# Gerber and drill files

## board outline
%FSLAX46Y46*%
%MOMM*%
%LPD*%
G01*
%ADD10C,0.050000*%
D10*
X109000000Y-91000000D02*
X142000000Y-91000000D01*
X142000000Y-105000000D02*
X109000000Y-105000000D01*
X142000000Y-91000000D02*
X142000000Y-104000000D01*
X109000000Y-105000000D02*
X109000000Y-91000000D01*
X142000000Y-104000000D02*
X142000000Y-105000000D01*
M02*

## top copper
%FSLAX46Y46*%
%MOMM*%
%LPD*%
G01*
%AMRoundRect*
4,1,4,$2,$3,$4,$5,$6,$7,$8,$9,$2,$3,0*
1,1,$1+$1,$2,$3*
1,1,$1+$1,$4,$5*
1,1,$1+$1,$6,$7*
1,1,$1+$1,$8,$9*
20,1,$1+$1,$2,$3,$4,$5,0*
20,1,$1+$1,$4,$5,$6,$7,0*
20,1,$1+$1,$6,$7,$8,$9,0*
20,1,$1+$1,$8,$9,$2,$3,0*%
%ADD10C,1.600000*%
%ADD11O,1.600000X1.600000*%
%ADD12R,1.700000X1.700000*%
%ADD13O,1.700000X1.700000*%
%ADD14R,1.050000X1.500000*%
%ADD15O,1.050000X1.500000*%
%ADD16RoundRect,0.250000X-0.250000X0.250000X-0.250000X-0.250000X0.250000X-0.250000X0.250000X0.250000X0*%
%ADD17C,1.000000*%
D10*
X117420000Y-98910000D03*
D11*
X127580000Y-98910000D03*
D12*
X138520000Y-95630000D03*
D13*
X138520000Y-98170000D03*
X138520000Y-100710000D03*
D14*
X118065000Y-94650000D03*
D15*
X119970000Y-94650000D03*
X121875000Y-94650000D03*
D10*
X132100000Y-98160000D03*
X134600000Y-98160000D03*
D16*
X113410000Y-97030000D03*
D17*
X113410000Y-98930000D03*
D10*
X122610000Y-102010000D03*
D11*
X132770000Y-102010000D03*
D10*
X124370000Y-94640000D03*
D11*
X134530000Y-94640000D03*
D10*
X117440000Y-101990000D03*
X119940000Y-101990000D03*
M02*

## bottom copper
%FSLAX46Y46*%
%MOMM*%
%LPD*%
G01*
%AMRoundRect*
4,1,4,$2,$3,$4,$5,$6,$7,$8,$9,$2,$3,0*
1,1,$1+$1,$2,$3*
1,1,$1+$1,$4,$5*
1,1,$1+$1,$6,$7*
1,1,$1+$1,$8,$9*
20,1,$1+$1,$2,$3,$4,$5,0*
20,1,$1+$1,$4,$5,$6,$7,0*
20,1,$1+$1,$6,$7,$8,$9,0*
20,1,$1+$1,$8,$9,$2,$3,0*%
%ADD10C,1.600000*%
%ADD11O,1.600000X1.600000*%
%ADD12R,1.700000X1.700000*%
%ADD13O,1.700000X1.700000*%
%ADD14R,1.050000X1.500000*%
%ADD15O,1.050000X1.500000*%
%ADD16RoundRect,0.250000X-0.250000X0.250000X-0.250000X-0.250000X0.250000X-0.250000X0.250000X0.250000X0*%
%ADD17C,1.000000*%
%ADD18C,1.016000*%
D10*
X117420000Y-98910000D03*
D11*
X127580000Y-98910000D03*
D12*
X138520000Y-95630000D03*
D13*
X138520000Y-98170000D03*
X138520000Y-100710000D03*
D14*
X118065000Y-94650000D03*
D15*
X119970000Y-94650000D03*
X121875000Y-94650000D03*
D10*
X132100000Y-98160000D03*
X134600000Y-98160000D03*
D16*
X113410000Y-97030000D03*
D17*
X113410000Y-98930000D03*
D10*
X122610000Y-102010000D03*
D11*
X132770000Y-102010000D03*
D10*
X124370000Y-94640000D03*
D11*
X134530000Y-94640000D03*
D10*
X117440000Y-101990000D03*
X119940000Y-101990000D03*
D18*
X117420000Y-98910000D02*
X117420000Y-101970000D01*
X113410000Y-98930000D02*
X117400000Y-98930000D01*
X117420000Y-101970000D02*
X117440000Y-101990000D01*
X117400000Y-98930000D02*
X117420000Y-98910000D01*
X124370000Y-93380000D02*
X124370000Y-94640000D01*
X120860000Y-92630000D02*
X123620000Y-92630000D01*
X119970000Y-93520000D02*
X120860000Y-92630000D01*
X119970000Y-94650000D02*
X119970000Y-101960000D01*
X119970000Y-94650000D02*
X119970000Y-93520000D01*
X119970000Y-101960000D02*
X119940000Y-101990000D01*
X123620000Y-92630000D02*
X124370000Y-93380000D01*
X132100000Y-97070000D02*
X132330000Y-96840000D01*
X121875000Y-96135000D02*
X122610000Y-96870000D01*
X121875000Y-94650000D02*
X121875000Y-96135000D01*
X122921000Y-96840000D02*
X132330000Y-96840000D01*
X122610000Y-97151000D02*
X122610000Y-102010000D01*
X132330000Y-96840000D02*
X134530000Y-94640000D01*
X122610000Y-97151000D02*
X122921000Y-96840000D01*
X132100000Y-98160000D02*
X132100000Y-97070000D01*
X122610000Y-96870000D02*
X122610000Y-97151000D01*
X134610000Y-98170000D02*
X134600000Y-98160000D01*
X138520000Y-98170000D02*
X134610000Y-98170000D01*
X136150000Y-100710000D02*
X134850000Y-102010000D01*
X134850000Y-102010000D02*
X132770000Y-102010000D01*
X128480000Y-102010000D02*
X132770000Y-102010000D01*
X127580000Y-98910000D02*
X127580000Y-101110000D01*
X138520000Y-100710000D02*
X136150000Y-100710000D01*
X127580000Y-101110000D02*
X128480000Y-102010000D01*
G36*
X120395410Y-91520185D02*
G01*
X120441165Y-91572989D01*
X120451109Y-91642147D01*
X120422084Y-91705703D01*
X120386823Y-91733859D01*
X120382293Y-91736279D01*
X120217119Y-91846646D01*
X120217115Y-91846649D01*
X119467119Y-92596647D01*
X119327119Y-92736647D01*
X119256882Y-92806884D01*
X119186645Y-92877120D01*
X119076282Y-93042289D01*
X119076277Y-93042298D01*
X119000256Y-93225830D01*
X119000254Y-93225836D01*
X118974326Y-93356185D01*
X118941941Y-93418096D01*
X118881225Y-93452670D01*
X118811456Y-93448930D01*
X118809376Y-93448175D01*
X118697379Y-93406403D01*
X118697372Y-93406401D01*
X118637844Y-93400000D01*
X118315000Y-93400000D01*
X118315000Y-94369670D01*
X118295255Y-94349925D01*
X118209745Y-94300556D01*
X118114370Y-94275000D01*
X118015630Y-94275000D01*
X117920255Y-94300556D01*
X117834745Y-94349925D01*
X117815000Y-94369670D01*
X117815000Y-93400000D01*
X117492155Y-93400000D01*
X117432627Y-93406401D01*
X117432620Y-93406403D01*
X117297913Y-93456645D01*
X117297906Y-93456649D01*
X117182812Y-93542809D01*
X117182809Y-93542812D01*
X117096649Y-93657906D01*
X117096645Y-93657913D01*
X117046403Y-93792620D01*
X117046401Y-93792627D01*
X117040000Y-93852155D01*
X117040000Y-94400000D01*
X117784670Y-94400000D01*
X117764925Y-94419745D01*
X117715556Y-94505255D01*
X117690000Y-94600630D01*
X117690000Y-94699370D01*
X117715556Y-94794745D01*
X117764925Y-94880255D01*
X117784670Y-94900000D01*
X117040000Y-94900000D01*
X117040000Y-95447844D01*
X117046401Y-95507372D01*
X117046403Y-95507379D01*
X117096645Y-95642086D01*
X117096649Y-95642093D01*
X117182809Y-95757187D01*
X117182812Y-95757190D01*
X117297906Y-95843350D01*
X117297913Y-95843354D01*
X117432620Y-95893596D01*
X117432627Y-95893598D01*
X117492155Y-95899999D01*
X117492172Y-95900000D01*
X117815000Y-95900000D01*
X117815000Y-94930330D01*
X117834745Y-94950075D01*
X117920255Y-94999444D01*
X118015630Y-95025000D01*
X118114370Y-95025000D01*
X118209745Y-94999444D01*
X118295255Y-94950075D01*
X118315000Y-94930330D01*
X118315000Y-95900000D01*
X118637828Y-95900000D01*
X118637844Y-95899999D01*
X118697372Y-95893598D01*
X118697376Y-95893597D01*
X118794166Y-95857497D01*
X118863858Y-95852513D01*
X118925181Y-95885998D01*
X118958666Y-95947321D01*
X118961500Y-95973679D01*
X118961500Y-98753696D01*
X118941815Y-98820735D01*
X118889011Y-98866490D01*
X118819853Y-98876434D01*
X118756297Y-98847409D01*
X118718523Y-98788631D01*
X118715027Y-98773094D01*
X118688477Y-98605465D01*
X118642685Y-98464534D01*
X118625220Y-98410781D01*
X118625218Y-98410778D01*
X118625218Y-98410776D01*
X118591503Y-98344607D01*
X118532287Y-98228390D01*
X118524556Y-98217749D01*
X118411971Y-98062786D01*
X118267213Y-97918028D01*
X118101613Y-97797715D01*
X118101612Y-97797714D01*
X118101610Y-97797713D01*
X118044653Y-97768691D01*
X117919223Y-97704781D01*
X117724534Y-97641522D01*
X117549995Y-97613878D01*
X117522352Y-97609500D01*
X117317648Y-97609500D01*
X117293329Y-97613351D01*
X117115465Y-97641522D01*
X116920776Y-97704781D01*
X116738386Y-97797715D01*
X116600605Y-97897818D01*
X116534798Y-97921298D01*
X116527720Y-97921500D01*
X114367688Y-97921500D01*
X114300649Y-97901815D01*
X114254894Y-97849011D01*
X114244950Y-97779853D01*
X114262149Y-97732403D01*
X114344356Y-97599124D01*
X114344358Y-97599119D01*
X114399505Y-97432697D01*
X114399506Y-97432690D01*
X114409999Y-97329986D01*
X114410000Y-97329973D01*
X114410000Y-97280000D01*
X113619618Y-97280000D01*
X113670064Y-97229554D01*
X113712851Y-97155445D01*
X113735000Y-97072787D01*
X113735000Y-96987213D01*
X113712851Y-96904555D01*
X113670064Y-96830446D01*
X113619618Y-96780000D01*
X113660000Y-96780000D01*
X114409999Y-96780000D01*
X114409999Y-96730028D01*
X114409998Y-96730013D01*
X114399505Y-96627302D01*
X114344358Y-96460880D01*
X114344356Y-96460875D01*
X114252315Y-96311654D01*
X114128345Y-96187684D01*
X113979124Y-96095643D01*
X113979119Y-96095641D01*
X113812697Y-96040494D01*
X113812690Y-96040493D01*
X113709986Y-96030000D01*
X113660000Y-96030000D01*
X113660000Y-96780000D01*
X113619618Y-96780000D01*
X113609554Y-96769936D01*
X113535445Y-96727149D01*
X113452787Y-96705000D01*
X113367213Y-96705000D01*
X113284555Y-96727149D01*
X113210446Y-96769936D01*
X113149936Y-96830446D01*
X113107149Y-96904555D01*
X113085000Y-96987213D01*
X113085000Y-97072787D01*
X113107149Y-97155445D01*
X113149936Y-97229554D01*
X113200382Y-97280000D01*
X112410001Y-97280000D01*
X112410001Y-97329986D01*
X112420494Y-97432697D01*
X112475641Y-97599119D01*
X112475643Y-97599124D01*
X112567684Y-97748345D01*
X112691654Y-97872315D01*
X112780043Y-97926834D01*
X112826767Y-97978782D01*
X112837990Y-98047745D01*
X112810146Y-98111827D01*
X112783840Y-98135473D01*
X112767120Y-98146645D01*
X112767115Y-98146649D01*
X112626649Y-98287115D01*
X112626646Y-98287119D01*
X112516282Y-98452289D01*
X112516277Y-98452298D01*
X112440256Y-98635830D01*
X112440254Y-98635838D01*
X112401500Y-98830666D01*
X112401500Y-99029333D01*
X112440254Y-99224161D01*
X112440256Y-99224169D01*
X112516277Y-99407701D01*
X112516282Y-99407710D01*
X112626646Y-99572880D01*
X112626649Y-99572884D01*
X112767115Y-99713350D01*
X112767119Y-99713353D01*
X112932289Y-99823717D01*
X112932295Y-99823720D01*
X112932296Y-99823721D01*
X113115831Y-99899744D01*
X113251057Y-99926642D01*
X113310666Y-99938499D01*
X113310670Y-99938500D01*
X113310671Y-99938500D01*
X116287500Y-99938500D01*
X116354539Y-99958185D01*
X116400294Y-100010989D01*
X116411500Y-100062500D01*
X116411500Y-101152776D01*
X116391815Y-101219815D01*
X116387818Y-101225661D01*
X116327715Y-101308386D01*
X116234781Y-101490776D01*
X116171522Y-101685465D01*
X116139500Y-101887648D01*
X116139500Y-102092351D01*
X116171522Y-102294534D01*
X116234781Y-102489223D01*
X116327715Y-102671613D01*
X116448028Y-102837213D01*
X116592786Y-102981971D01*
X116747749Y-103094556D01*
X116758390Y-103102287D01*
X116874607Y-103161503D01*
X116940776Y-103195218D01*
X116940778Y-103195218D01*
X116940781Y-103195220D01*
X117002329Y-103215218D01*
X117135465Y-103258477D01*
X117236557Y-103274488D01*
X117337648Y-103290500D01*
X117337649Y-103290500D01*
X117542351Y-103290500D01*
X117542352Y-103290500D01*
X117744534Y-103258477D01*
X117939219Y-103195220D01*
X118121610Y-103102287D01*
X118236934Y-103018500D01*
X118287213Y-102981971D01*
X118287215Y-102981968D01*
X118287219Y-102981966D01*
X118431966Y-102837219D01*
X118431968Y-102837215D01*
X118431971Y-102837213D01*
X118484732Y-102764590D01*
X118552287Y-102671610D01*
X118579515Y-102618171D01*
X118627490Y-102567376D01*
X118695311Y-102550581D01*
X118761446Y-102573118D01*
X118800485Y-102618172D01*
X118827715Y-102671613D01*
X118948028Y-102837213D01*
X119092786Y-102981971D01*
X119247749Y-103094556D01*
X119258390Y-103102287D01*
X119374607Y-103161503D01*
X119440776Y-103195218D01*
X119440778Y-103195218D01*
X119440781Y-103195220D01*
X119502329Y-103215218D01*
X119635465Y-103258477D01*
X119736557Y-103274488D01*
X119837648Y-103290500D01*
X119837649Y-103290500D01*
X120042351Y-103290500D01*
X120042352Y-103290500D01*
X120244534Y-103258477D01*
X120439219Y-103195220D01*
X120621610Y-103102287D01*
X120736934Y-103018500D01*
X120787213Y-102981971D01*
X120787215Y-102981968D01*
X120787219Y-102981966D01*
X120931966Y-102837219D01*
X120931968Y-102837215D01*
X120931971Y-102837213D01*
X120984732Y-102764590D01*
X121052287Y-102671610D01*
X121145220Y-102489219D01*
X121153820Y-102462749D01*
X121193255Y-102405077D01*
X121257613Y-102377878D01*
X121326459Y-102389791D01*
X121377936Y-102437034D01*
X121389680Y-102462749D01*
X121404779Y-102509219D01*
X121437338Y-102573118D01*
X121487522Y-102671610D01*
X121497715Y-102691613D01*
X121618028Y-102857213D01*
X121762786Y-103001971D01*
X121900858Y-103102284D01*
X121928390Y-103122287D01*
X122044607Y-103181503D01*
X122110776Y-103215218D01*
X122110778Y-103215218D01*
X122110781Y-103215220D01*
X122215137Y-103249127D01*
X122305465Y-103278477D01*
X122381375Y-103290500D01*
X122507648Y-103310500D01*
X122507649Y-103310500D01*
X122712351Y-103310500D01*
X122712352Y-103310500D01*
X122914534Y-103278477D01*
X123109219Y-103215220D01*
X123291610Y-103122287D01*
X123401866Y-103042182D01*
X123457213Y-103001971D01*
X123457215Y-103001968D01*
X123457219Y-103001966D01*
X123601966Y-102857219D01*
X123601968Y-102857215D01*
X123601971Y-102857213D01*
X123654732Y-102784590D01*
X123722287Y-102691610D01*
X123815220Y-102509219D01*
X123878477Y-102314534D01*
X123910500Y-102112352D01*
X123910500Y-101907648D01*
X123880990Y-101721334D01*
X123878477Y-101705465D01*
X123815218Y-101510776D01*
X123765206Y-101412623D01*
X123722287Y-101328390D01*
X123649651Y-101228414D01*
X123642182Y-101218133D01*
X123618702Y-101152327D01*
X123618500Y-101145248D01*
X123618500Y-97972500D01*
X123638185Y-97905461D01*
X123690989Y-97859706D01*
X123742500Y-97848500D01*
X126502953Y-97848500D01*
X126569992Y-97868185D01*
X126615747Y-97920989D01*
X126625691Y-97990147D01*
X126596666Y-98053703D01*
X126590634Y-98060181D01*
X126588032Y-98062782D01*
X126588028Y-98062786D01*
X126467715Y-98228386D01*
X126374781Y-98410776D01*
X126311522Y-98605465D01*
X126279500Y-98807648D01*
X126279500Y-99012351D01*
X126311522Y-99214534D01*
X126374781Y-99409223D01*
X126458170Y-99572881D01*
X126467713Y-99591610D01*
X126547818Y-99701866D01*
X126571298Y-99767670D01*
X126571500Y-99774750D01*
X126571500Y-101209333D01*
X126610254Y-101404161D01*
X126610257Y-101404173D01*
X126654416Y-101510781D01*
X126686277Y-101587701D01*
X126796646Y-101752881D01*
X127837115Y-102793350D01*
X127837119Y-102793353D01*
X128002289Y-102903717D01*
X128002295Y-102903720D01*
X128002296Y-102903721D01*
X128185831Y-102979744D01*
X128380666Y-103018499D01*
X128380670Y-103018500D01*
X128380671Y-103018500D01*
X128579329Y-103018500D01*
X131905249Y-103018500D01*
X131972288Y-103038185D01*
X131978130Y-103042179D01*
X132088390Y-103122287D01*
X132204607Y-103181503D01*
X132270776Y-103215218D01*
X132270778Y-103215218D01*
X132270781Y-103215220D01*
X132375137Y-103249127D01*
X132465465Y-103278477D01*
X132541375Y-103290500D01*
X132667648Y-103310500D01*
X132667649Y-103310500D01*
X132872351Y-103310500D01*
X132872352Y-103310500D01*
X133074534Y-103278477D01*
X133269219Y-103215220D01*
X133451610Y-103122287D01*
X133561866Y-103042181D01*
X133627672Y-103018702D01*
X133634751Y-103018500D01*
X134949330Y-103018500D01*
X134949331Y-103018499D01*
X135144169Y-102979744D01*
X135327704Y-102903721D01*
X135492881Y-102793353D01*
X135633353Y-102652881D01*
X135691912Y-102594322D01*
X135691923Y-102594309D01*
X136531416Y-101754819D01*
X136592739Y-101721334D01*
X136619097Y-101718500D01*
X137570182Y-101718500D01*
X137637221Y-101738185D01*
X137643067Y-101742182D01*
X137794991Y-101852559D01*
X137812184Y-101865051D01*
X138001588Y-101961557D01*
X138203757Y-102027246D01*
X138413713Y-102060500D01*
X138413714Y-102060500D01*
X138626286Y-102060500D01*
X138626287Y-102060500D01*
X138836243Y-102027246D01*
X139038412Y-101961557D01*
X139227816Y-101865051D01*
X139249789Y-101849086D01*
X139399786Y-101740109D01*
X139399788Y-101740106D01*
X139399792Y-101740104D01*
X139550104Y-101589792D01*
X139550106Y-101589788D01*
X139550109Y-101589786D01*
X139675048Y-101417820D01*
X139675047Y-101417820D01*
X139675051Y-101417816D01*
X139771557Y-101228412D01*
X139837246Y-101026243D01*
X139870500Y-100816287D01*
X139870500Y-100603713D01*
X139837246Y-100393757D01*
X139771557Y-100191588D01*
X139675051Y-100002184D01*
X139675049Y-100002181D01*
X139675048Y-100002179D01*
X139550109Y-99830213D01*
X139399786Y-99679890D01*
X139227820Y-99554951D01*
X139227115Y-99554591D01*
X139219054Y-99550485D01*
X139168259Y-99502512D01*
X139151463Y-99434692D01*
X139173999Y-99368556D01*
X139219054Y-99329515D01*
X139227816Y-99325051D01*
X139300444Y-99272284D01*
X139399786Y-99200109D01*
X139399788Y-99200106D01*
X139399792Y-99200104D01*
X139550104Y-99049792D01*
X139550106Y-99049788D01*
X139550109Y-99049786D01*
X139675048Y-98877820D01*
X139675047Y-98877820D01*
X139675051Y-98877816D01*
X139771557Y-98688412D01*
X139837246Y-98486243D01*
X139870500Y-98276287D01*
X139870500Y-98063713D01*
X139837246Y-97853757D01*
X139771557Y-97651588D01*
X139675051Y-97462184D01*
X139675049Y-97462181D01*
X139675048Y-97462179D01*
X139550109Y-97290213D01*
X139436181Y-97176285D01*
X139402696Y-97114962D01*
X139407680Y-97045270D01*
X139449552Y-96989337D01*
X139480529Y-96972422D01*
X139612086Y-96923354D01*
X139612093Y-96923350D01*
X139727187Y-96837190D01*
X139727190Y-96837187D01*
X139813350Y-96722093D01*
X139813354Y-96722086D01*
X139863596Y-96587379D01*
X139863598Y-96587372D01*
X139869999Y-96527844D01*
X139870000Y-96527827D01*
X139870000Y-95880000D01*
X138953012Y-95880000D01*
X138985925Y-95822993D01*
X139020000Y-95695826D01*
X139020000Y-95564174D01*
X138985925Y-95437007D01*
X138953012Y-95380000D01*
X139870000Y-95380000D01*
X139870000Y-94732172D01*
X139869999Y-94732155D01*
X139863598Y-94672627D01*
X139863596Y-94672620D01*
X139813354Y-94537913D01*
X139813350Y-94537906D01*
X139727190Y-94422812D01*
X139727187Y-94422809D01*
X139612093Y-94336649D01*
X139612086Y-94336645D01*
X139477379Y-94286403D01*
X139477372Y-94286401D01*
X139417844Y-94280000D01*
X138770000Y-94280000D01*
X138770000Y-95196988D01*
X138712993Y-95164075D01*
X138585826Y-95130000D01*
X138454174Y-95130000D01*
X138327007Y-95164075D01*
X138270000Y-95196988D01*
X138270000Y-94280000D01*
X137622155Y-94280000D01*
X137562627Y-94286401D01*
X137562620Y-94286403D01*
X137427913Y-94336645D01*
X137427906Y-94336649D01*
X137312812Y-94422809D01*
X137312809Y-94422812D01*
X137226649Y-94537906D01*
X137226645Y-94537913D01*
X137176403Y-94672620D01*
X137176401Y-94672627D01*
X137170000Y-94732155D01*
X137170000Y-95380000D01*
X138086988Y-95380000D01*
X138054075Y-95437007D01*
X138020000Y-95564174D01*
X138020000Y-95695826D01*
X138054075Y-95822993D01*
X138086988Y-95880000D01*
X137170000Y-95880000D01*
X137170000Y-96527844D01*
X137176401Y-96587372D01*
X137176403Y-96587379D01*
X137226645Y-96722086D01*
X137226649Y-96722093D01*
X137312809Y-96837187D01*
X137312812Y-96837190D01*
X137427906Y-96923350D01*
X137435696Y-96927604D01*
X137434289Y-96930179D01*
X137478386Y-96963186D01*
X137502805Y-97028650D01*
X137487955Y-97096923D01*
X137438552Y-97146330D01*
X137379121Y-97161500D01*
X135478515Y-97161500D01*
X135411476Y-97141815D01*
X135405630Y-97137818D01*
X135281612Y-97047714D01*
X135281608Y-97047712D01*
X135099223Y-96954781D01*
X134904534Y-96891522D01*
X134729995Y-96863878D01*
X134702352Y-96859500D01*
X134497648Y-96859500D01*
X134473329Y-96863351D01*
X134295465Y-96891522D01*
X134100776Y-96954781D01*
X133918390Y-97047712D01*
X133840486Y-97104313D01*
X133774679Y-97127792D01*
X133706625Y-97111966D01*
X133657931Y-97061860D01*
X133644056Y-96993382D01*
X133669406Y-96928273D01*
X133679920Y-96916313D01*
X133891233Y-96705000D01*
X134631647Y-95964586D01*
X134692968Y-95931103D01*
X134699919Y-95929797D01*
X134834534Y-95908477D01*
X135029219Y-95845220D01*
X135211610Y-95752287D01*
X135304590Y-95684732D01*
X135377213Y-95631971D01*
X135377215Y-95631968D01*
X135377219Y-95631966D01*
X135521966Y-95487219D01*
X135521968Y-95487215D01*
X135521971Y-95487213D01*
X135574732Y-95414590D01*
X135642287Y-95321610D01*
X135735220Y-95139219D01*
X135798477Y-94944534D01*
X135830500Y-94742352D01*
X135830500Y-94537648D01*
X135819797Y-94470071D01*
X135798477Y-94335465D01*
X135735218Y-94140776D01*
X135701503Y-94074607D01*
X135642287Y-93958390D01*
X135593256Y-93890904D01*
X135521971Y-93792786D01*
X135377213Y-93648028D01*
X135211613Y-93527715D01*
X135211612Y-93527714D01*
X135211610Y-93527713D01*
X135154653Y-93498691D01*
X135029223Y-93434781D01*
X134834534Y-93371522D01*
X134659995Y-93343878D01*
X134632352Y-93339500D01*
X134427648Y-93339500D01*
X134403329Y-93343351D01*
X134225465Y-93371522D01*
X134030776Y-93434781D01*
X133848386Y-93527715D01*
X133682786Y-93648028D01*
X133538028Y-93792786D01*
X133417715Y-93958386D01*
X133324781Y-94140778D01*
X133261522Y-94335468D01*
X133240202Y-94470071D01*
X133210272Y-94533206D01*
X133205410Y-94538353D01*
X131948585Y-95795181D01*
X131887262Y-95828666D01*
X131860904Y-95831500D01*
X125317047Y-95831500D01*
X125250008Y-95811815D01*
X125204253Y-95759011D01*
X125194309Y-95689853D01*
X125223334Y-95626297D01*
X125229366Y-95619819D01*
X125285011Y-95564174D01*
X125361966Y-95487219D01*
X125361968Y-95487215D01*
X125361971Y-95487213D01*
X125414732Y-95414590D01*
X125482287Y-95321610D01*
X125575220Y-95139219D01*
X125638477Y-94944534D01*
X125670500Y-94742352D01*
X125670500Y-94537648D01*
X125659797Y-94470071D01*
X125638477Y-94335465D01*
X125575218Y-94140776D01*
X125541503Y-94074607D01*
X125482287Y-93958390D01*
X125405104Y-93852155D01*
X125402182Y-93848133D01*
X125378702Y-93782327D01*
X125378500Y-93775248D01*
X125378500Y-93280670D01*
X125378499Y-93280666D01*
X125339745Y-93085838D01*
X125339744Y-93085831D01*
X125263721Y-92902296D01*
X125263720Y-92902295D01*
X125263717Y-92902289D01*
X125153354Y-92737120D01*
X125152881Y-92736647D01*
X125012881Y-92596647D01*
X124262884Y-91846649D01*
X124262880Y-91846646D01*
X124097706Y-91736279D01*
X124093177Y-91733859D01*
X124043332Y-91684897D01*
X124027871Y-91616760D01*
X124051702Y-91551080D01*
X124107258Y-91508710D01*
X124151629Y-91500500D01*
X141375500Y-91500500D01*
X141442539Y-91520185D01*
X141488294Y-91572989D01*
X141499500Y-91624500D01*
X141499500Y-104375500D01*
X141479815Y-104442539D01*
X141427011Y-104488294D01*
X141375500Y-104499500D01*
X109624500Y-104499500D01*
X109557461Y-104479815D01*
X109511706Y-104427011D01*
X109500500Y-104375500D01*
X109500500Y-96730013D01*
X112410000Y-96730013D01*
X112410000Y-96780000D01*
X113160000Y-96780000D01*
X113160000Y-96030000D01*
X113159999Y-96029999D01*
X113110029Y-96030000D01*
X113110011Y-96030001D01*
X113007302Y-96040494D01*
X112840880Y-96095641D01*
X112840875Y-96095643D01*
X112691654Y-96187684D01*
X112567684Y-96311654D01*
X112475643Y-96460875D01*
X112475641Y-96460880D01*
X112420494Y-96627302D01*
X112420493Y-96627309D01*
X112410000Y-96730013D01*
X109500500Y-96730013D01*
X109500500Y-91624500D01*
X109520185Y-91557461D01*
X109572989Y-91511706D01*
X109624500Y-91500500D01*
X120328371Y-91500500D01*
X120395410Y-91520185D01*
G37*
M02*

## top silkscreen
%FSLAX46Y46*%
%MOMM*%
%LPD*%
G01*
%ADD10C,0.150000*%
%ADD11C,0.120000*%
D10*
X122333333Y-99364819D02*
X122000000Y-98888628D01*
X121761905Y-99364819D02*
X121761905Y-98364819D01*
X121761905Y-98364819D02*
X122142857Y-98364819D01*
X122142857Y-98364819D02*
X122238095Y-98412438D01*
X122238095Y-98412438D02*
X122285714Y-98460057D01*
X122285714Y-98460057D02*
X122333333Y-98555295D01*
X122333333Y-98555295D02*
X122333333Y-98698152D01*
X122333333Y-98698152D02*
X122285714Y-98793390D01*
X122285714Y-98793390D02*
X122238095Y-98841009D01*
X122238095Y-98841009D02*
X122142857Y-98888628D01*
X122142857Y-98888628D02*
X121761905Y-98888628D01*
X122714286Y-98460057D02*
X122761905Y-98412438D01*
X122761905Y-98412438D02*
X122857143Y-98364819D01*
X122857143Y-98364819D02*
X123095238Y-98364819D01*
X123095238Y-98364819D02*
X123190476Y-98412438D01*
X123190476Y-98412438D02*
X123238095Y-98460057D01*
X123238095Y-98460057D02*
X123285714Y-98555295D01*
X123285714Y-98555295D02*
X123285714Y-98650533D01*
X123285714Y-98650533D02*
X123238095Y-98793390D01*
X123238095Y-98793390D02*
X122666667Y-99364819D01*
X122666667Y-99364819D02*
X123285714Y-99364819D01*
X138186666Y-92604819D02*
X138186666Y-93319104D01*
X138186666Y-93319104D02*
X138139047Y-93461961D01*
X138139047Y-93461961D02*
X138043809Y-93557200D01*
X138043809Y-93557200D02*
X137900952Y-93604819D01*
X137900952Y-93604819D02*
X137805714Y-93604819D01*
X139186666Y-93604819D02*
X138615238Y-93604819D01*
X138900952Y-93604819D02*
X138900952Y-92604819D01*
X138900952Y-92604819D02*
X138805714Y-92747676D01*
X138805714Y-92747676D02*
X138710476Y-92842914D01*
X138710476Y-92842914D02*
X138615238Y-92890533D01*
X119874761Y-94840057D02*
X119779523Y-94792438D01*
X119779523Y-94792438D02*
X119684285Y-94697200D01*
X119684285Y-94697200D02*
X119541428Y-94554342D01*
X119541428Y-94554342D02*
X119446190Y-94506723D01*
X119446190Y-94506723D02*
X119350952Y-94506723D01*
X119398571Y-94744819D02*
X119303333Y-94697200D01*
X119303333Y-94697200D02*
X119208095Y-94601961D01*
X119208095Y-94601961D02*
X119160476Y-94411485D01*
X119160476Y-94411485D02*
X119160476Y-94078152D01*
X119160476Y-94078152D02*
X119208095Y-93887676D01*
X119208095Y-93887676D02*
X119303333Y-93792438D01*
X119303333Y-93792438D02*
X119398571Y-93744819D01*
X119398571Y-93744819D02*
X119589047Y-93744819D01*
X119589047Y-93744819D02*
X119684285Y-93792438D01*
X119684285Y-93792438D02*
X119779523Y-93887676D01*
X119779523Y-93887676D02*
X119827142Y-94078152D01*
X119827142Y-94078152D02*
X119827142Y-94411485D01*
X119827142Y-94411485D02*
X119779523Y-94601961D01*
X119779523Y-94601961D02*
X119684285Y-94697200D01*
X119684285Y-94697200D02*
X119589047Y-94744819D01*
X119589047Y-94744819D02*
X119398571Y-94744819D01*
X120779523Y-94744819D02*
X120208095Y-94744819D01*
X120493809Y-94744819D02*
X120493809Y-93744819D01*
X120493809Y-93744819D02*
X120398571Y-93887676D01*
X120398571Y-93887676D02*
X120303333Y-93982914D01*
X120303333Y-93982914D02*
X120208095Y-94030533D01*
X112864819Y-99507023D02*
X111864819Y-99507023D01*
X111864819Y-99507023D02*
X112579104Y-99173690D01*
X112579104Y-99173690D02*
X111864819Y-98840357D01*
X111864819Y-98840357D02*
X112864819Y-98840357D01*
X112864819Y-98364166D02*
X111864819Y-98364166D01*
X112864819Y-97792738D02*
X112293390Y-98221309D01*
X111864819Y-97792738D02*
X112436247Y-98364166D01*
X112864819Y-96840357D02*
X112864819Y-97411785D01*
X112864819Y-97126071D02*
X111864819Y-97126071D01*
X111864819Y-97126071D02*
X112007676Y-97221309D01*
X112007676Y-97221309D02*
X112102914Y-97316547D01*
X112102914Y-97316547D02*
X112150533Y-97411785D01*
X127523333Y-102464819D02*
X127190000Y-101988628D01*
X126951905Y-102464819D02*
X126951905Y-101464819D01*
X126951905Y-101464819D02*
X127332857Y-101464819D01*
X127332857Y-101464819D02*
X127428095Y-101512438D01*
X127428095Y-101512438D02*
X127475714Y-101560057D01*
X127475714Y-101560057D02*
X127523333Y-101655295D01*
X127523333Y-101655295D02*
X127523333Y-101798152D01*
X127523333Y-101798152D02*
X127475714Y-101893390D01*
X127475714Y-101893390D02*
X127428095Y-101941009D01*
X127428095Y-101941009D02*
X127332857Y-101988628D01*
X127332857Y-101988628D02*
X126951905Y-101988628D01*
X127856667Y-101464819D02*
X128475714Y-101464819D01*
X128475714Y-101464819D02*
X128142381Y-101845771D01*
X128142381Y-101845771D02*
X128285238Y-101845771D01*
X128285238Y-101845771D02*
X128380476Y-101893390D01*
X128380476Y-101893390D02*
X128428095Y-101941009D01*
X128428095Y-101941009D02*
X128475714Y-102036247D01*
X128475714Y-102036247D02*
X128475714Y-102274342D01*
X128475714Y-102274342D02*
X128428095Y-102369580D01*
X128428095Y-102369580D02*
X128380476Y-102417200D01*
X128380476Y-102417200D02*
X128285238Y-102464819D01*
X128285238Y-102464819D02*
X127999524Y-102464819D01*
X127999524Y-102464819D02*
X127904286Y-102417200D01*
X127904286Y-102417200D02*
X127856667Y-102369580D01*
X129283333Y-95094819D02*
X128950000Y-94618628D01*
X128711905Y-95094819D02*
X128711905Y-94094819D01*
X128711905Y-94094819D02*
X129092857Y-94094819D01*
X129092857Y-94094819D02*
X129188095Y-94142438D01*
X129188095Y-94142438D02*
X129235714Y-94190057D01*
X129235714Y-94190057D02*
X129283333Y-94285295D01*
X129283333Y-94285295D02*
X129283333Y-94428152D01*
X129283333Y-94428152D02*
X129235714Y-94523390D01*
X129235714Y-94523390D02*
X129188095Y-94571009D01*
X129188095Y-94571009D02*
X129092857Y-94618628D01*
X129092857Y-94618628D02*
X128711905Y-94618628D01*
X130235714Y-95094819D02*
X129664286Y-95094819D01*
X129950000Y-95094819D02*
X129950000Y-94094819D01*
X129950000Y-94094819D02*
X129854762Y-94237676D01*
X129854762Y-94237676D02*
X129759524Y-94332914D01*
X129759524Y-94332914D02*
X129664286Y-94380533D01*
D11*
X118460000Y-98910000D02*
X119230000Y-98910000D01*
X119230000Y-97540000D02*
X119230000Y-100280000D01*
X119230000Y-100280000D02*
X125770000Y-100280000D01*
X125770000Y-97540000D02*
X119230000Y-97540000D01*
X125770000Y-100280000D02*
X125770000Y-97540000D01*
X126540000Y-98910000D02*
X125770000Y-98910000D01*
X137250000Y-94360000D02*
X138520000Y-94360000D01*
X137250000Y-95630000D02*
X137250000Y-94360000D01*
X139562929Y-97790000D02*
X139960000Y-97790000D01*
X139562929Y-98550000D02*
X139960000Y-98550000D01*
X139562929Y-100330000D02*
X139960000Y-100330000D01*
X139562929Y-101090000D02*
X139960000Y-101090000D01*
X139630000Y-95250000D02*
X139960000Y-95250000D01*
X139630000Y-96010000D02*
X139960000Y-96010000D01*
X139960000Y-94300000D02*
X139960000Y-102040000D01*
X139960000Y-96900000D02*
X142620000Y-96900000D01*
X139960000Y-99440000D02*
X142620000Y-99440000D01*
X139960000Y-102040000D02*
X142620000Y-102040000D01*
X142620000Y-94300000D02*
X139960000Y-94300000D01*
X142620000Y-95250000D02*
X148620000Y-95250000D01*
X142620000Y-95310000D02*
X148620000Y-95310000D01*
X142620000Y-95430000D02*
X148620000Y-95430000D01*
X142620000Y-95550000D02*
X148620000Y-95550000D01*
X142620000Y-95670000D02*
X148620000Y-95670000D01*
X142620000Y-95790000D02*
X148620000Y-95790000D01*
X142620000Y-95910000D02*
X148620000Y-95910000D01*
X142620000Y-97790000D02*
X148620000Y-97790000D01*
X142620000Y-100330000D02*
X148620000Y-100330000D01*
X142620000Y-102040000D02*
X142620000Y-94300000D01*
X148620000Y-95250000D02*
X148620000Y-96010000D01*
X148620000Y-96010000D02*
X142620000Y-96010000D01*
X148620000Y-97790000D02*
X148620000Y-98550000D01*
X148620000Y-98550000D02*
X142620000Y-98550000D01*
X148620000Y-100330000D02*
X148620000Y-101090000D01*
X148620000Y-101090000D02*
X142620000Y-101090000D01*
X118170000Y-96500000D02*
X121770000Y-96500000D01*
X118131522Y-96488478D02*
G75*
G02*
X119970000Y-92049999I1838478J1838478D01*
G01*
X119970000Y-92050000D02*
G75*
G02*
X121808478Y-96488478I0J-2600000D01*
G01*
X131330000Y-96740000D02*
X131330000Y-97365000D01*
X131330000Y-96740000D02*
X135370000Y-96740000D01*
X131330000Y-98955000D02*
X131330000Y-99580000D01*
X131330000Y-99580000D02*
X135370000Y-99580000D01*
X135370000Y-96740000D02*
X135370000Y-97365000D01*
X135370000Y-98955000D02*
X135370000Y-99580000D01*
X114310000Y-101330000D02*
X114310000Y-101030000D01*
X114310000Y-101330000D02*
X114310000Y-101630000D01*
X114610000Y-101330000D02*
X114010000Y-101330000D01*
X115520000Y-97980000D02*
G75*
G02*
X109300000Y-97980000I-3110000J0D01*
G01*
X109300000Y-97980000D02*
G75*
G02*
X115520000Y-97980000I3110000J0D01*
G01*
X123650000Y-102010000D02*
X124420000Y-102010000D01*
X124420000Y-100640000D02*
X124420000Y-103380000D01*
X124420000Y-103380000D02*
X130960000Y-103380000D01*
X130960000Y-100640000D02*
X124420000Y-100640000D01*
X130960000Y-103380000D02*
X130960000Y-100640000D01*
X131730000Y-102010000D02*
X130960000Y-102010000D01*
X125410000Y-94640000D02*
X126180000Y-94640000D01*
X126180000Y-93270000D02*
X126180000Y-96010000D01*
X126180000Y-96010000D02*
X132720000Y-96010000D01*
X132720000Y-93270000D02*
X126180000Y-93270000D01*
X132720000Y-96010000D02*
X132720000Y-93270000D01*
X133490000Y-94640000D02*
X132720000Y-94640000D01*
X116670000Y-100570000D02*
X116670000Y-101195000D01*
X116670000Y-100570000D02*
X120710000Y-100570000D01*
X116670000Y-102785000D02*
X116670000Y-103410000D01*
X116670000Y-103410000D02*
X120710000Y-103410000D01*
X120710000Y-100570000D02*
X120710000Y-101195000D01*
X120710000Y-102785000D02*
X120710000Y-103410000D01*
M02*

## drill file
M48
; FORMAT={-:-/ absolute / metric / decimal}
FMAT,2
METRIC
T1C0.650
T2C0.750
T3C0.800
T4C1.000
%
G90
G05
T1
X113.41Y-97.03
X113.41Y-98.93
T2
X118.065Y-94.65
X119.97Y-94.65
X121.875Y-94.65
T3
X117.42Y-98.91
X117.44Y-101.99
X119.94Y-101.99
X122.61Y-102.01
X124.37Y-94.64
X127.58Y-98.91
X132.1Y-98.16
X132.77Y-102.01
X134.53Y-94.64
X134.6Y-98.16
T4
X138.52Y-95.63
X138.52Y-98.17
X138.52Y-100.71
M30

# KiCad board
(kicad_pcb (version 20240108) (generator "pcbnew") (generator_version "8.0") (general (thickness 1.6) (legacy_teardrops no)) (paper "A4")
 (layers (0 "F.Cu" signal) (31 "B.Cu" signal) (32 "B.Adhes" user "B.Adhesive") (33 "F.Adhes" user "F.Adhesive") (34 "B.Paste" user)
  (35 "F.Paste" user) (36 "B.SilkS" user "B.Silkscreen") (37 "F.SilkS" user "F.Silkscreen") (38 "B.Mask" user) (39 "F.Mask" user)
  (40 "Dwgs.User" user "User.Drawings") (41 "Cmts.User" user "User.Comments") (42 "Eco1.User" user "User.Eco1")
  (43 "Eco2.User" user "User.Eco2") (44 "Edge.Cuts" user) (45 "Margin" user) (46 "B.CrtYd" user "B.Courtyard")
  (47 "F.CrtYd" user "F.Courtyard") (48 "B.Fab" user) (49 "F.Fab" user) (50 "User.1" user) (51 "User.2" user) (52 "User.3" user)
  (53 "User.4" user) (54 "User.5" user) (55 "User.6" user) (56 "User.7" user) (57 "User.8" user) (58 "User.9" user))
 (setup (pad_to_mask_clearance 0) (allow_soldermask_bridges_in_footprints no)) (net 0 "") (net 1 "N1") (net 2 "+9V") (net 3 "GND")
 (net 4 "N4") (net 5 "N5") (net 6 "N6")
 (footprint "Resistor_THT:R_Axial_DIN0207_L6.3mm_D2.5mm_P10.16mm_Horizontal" (layer "F.Cu") (at 117.42 98.91)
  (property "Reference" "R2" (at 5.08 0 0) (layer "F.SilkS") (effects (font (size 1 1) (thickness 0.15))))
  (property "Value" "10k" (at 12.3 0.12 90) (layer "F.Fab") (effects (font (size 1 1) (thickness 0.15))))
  (fp_line (start 1.04 0) (end 1.81 0) (stroke (width 0.12) (type solid)) (layer "F.SilkS"))
  (fp_line (start 1.81 -1.37) (end 1.81 1.37) (stroke (width 0.12) (type solid)) (layer "F.SilkS"))
  (fp_line (start 1.81 1.37) (end 8.35 1.37) (stroke (width 0.12) (type solid)) (layer "F.SilkS"))
  (fp_line (start 8.35 -1.37) (end 1.81 -1.37) (stroke (width 0.12) (type solid)) (layer "F.SilkS"))
  (fp_line (start 8.35 1.37) (end 8.35 -1.37) (stroke (width 0.12) (type solid)) (layer "F.SilkS"))
  (fp_line (start 9.12 0) (end 8.35 0) (stroke (width 0.12) (type solid)) (layer "F.SilkS"))
  (pad "1" thru_hole circle (at 0 0) (size 1.6 1.6) (drill 0.8) (layers "*.Cu" "*.Mask") (remove_unused_layers no) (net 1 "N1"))
  (pad "2" thru_hole oval (at 10.16 0) (size 1.6 1.6) (drill 0.8) (layers "*.Cu" "*.Mask") (remove_unused_layers no) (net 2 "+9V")))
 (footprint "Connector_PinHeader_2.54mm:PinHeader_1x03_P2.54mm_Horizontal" (layer "F.Cu") (at 138.52 95.63)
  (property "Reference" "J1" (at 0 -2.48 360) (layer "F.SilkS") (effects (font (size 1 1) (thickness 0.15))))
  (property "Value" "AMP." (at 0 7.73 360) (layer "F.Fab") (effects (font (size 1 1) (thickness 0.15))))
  (fp_line (start -1.27 -1.27) (end 0 -1.27) (stroke (width 0.12) (type solid)) (layer "F.SilkS"))
  (fp_line (start -1.27 0) (end -1.27 -1.27) (stroke (width 0.12) (type solid)) (layer "F.SilkS"))
  (fp_line (start 1.042929 2.16) (end 1.44 2.16) (stroke (width 0.12) (type solid)) (layer "F.SilkS"))
  (fp_line (start 1.042929 2.92) (end 1.44 2.92) (stroke (width 0.12) (type solid)) (layer "F.SilkS"))
  (fp_line (start 1.042929 4.7) (end 1.44 4.7) (stroke (width 0.12) (type solid)) (layer "F.SilkS"))
  (fp_line (start 1.042929 5.46) (end 1.44 5.46) (stroke (width 0.12) (type solid)) (layer "F.SilkS"))
  (fp_line (start 1.11 -0.38) (end 1.44 -0.38) (stroke (width 0.12) (type solid)) (layer "F.SilkS"))
  (fp_line (start 1.11 0.38) (end 1.44 0.38) (stroke (width 0.12) (type solid)) (layer "F.SilkS"))
  (fp_line (start 1.44 -1.33) (end 1.44 6.41) (stroke (width 0.12) (type solid)) (layer "F.SilkS"))
  (fp_line (start 1.44 1.27) (end 4.1 1.27) (stroke (width 0.12) (type solid)) (layer "F.SilkS"))
  (fp_line (start 1.44 3.81) (end 4.1 3.81) (stroke (width 0.12) (type solid)) (layer "F.SilkS"))
  (fp_line (start 1.44 6.41) (end 4.1 6.41) (stroke (width 0.12) (type solid)) (layer "F.SilkS"))
  (fp_line (start 4.1 -1.33) (end 1.44 -1.33) (stroke (width 0.12) (type solid)) (layer "F.SilkS"))
  (fp_line (start 4.1 -0.38) (end 10.1 -0.38) (stroke (width 0.12) (type solid)) (layer "F.SilkS"))
  (fp_line (start 4.1 -0.32) (end 10.1 -0.32) (stroke (width 0.12) (type solid)) (layer "F.SilkS"))
  (fp_line (start 4.1 -0.2) (end 10.1 -0.2) (stroke (width 0.12) (type solid)) (layer "F.SilkS"))
  (fp_line (start 4.1 -0.08) (end 10.1 -0.08) (stroke (width 0.12) (type solid)) (layer "F.SilkS"))
  (fp_line (start 4.1 0.04) (end 10.1 0.04) (stroke (width 0.12) (type solid)) (layer "F.SilkS"))
  (fp_line (start 4.1 0.16) (end 10.1 0.16) (stroke (width 0.12) (type solid)) (layer "F.SilkS"))
  (fp_line (start 4.1 0.28) (end 10.1 0.28) (stroke (width 0.12) (type solid)) (layer "F.SilkS"))
  (fp_line (start 4.1 2.16) (end 10.1 2.16) (stroke (width 0.12) (type solid)) (layer "F.SilkS"))
  (fp_line (start 4.1 4.7) (end 10.1 4.7) (stroke (width 0.12) (type solid)) (layer "F.SilkS"))
  (fp_line (start 4.1 6.41) (end 4.1 -1.33) (stroke (width 0.12) (type solid)) (layer "F.SilkS"))
  (fp_line (start 10.1 -0.38) (end 10.1 0.38) (stroke (width 0.12) (type solid)) (layer "F.SilkS"))
  (fp_line (start 10.1 0.38) (end 4.1 0.38) (stroke (width 0.12) (type solid)) (layer "F.SilkS"))
  (fp_line (start 10.1 2.16) (end 10.1 2.92) (stroke (width 0.12) (type solid)) (layer "F.SilkS"))
  (fp_line (start 10.1 2.92) (end 4.1 2.92) (stroke (width 0.12) (type solid)) (layer "F.SilkS"))
  (fp_line (start 10.1 4.7) (end 10.1 5.46) (stroke (width 0.12) (type solid)) (layer "F.SilkS"))
  (fp_line (start 10.1 5.46) (end 4.1 5.46) (stroke (width 0.12) (type solid)) (layer "F.SilkS"))
  (pad "1" thru_hole rect (at 0 0) (size 1.7 1.7) (drill 1) (layers "*.Cu" "*.Mask") (remove_unused_layers no) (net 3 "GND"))
  (pad "2" thru_hole oval (at 0 2.54) (size 1.7 1.7) (drill 1) (layers "*.Cu" "*.Mask") (remove_unused_layers no) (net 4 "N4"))
  (pad "3" thru_hole oval (at 0 5.08) (size 1.7 1.7) (drill 1) (layers "*.Cu" "*.Mask") (remove_unused_layers no) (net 2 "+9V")))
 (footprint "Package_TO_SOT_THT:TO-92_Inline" (layer "F.Cu") (at 118.7 94.65)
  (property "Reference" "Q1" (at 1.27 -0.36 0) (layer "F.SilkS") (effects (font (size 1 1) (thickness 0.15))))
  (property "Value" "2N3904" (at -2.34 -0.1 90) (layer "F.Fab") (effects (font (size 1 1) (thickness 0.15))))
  (fp_line (start -0.53 1.85) (end 3.07 1.85) (stroke (width 0.12) (type solid)) (layer "F.SilkS"))
  (fp_arc (start -0.568478 1.838478) (mid -1.132087 -0.994977) (end 1.27 -2.6) (stroke (width 0.12) (type solid)) (layer "F.SilkS"))
  (fp_arc (start 1.27 -2.6) (mid 3.672087 -0.994977) (end 3.108478 1.838478) (stroke (width 0.12) (type solid)) (layer "F.SilkS"))
  (pad "1" thru_hole rect (at -0.635 0) (size 1.05 1.5) (drill 0.75) (layers "*.Cu" "*.Mask") (remove_unused_layers no) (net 3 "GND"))
  (pad "2" thru_hole oval (at 1.27 0) (size 1.05 1.5) (drill 0.75) (layers "*.Cu" "*.Mask") (remove_unused_layers no) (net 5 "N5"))
  (pad "3" thru_hole oval (at 3.175 0) (size 1.05 1.5) (drill 0.75) (layers "*.Cu" "*.Mask") (remove_unused_layers no) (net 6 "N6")))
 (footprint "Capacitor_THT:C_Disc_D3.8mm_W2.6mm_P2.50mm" (layer "F.Cu") (at 132.1 98.16)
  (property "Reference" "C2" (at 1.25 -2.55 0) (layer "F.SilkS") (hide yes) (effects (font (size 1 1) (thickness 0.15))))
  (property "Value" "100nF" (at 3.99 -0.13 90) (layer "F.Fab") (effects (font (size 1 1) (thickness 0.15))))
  (fp_line (start -0.77 -1.42) (end -0.77 -0.795) (stroke (width 0.12) (type solid)) (layer "F.SilkS"))
  (fp_line (start -0.77 -1.42) (end 3.27 -1.42) (stroke (width 0.12) (type solid)) (layer "F.SilkS"))
  (fp_line (start -0.77 0.795) (end -0.77 1.42) (stroke (width 0.12) (type solid)) (layer "F.SilkS"))
  (fp_line (start -0.77 1.42) (end 3.27 1.42) (stroke (width 0.12) (type solid)) (layer "F.SilkS"))
  (fp_line (start 3.27 -1.42) (end 3.27 -0.795) (stroke (width 0.12) (type solid)) (layer "F.SilkS"))
  (fp_line (start 3.27 0.795) (end 3.27 1.42) (stroke (width 0.12) (type solid)) (layer "F.SilkS"))
  (pad "1" thru_hole circle (at 0 0) (size 1.6 1.6) (drill 0.8) (layers "*.Cu" "*.Mask") (remove_unused_layers no) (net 6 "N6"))
  (pad "2" thru_hole circle (at 2.5 0) (size 1.6 1.6) (drill 0.8) (layers "*.Cu" "*.Mask") (remove_unused_layers no) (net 4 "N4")))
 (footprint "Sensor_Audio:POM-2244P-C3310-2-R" (layer "F.Cu") (at 113.41 97.03 -90)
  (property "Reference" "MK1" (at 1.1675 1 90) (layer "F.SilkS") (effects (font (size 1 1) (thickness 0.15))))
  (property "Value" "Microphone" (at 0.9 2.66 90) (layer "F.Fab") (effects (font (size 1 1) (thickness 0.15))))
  (fp_line (start 4.3 -0.9) (end 4 -0.9) (stroke (width 0.12) (type default)) (layer "F.SilkS"))
  (fp_line (start 4.3 -0.9) (end 4.6 -0.9) (stroke (width 0.12) (type default)) (layer "F.SilkS"))
  (fp_line (start 4.3 -1.2) (end 4.3 -0.6) (stroke (width 0.12) (type default)) (layer "F.SilkS"))
  (fp_circle (center 0.95 1) (end 4.06 1) (stroke (width 0.12) (type default)) (fill none) (layer "F.SilkS"))
  (pad "1" thru_hole roundrect (at 0 0 270) (size 1 1) (drill 0.65) (layers "*.Cu" "*.Mask") (remove_unused_layers no)
   (roundrect_rratio 0.25) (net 3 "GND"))
  (pad "2" thru_hole circle (at 1.9 0 270) (size 1 1) (drill 0.65) (layers "*.Cu" "*.Mask") (remove_unused_layers no) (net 1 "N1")))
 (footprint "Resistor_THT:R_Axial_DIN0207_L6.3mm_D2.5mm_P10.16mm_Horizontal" (layer "F.Cu") (at 122.61 102.01)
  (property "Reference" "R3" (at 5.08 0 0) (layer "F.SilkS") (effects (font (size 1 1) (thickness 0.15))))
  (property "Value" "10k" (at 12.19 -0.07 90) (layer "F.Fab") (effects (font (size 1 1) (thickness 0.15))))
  (fp_line (start 1.04 0) (end 1.81 0) (stroke (width 0.12) (type solid)) (layer "F.SilkS"))
  (fp_line (start 1.81 -1.37) (end 1.81 1.37) (stroke (width 0.12) (type solid)) (layer "F.SilkS"))
  (fp_line (start 1.81 1.37) (end 8.35 1.37) (stroke (width 0.12) (type solid)) (layer "F.SilkS"))
  (fp_line (start 8.35 -1.37) (end 1.81 -1.37) (stroke (width 0.12) (type solid)) (layer "F.SilkS"))
  (fp_line (start 8.35 1.37) (end 8.35 -1.37) (stroke (width 0.12) (type solid)) (layer "F.SilkS"))
  (fp_line (start 9.12 0) (end 8.35 0) (stroke (width 0.12) (type solid)) (layer "F.SilkS"))
  (pad "1" thru_hole circle (at 0 0) (size 1.6 1.6) (drill 0.8) (layers "*.Cu" "*.Mask") (remove_unused_layers no) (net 6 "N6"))
  (pad "2" thru_hole oval (at 10.16 0) (size 1.6 1.6) (drill 0.8) (layers "*.Cu" "*.Mask") (remove_unused_layers no) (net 2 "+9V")))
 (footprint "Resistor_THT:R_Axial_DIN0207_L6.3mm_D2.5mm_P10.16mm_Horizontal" (layer "F.Cu") (at 124.37 94.64)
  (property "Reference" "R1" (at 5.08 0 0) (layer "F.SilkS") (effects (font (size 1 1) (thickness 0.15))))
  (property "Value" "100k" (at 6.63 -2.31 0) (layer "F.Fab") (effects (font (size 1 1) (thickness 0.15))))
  (fp_line (start 1.04 0) (end 1.81 0) (stroke (width 0.12) (type solid)) (layer "F.SilkS"))
  (fp_line (start 1.81 -1.37) (end 1.81 1.37) (stroke (width 0.12) (type solid)) (layer "F.SilkS"))
  (fp_line (start 1.81 1.37) (end 8.35 1.37) (stroke (width 0.12) (type solid)) (layer "F.SilkS"))
  (fp_line (start 8.35 -1.37) (end 1.81 -1.37) (stroke (width 0.12) (type solid)) (layer "F.SilkS"))
  (fp_line (start 8.35 1.37) (end 8.35 -1.37) (stroke (width 0.12) (type solid)) (layer "F.SilkS"))
  (fp_line (start 9.12 0) (end 8.35 0) (stroke (width 0.12) (type solid)) (layer "F.SilkS"))
  (pad "1" thru_hole circle (at 0 0) (size 1.6 1.6) (drill 0.8) (layers "*.Cu" "*.Mask") (remove_unused_layers no) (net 5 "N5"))
  (pad "2" thru_hole oval (at 10.16 0) (size 1.6 1.6) (drill 0.8) (layers "*.Cu" "*.Mask") (remove_unused_layers no) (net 6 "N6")))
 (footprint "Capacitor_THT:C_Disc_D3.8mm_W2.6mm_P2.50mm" (layer "F.Cu") (at 117.44 101.99)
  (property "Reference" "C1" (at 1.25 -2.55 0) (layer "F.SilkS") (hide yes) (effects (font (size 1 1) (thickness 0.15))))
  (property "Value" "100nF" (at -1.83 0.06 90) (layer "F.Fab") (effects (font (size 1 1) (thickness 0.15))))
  (fp_line (start -0.77 -1.42) (end -0.77 -0.795) (stroke (width 0.12) (type solid)) (layer "F.SilkS"))
  (fp_line (start -0.77 -1.42) (end 3.27 -1.42) (stroke (width 0.12) (type solid)) (layer "F.SilkS"))
  (fp_line (start -0.77 0.795) (end -0.77 1.42) (stroke (width 0.12) (type solid)) (layer "F.SilkS"))
  (fp_line (start -0.77 1.42) (end 3.27 1.42) (stroke (width 0.12) (type solid)) (layer "F.SilkS"))
  (fp_line (start 3.27 -1.42) (end 3.27 -0.795) (stroke (width 0.12) (type solid)) (layer "F.SilkS"))
  (fp_line (start 3.27 0.795) (end 3.27 1.42) (stroke (width 0.12) (type solid)) (layer "F.SilkS"))
  (pad "1" thru_hole circle (at 0 0) (size 1.6 1.6) (drill 0.8) (layers "*.Cu" "*.Mask") (remove_unused_layers no) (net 1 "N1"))
  (pad "2" thru_hole circle (at 2.5 0) (size 1.6 1.6) (drill 0.8) (layers "*.Cu" "*.Mask") (remove_unused_layers no) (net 5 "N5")))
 (gr_line (start 109 91) (end 142 91) (stroke (width 0.05) (type default)) (layer "Edge.Cuts"))
 (gr_line (start 142 105) (end 109 105) (stroke (width 0.05) (type default)) (layer "Edge.Cuts"))
 (gr_line (start 142 91) (end 142 104) (stroke (width 0.05) (type default)) (layer "Edge.Cuts"))
 (gr_line (start 109 105) (end 109 91) (stroke (width 0.05) (type default)) (layer "Edge.Cuts"))
 (gr_line (start 142 104) (end 142 105) (stroke (width 0.05) (type default)) (layer "Edge.Cuts"))
 (segment (start 117.42 98.91) (end 117.42 101.97) (width 1.016) (layer "B.Cu") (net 1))
 (segment (start 113.41 98.93) (end 117.4 98.93) (width 1.016) (layer "B.Cu") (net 1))
 (segment (start 117.42 101.97) (end 117.44 101.99) (width 1.016) (layer "B.Cu") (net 1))
 (segment (start 117.4 98.93) (end 117.42 98.91) (width 1.016) (layer "B.Cu") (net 1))
 (segment (start 124.37 93.38) (end 124.37 94.64) (width 1.016) (layer "B.Cu") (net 5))
 (segment (start 120.86 92.63) (end 123.62 92.63) (width 1.016) (layer "B.Cu") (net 5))
 (segment (start 119.97 93.52) (end 120.86 92.63) (width 1.016) (layer "B.Cu") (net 5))
 (segment (start 119.97 94.65) (end 119.97 101.96) (width 1.016) (layer "B.Cu") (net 5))
 (segment (start 119.97 94.65) (end 119.97 93.52) (width 1.016) (layer "B.Cu") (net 5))
 (segment (start 119.97 101.96) (end 119.94 101.99) (width 1.016) (layer "B.Cu") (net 5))
 (segment (start 123.62 92.63) (end 124.37 93.38) (width 1.016) (layer "B.Cu") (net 5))
 (segment (start 132.1 97.07) (end 132.33 96.84) (width 1.016) (layer "B.Cu") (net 6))
 (segment (start 121.875 96.135) (end 122.61 96.87) (width 1.016) (layer "B.Cu") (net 6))
 (segment (start 121.875 94.65) (end 121.875 96.135) (width 1.016) (layer "B.Cu") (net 6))
 (segment (start 122.921 96.84) (end 132.33 96.84) (width 1.016) (layer "B.Cu") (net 6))
 (segment (start 122.61 97.151) (end 122.61 102.01) (width 1.016) (layer "B.Cu") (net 6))
 (segment (start 132.33 96.84) (end 134.53 94.64) (width 1.016) (layer "B.Cu") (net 6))
 (segment (start 122.61 97.151) (end 122.921 96.84) (width 1.016) (layer "B.Cu") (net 6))
 (segment (start 132.1 98.16) (end 132.1 97.07) (width 1.016) (layer "B.Cu") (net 6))
 (segment (start 122.61 96.87) (end 122.61 97.151) (width 1.016) (layer "B.Cu") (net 6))
 (segment (start 134.61 98.17) (end 134.6 98.16) (width 1.016) (layer "B.Cu") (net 4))
 (segment (start 138.52 98.17) (end 134.61 98.17) (width 1.016) (layer "B.Cu") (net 4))
 (segment (start 136.15 100.71) (end 134.85 102.01) (width 1.016) (layer "B.Cu") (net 2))
 (segment (start 134.85 102.01) (end 132.77 102.01) (width 1.016) (layer "B.Cu") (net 2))
 (segment (start 128.48 102.01) (end 132.77 102.01) (width 1.016) (layer "B.Cu") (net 2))
 (segment (start 127.58 98.91) (end 127.58 101.11) (width 1.016) (layer "B.Cu") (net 2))
 (segment (start 138.52 100.71) (end 136.15 100.71) (width 1.016) (layer "B.Cu") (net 2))
 (segment (start 127.58 101.11) (end 128.48 102.01) (width 1.016) (layer "B.Cu") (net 2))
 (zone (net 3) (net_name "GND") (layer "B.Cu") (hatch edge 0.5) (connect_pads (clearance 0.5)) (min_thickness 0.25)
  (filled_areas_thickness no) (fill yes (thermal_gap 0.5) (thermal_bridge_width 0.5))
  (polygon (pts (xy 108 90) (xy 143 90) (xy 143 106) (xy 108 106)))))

